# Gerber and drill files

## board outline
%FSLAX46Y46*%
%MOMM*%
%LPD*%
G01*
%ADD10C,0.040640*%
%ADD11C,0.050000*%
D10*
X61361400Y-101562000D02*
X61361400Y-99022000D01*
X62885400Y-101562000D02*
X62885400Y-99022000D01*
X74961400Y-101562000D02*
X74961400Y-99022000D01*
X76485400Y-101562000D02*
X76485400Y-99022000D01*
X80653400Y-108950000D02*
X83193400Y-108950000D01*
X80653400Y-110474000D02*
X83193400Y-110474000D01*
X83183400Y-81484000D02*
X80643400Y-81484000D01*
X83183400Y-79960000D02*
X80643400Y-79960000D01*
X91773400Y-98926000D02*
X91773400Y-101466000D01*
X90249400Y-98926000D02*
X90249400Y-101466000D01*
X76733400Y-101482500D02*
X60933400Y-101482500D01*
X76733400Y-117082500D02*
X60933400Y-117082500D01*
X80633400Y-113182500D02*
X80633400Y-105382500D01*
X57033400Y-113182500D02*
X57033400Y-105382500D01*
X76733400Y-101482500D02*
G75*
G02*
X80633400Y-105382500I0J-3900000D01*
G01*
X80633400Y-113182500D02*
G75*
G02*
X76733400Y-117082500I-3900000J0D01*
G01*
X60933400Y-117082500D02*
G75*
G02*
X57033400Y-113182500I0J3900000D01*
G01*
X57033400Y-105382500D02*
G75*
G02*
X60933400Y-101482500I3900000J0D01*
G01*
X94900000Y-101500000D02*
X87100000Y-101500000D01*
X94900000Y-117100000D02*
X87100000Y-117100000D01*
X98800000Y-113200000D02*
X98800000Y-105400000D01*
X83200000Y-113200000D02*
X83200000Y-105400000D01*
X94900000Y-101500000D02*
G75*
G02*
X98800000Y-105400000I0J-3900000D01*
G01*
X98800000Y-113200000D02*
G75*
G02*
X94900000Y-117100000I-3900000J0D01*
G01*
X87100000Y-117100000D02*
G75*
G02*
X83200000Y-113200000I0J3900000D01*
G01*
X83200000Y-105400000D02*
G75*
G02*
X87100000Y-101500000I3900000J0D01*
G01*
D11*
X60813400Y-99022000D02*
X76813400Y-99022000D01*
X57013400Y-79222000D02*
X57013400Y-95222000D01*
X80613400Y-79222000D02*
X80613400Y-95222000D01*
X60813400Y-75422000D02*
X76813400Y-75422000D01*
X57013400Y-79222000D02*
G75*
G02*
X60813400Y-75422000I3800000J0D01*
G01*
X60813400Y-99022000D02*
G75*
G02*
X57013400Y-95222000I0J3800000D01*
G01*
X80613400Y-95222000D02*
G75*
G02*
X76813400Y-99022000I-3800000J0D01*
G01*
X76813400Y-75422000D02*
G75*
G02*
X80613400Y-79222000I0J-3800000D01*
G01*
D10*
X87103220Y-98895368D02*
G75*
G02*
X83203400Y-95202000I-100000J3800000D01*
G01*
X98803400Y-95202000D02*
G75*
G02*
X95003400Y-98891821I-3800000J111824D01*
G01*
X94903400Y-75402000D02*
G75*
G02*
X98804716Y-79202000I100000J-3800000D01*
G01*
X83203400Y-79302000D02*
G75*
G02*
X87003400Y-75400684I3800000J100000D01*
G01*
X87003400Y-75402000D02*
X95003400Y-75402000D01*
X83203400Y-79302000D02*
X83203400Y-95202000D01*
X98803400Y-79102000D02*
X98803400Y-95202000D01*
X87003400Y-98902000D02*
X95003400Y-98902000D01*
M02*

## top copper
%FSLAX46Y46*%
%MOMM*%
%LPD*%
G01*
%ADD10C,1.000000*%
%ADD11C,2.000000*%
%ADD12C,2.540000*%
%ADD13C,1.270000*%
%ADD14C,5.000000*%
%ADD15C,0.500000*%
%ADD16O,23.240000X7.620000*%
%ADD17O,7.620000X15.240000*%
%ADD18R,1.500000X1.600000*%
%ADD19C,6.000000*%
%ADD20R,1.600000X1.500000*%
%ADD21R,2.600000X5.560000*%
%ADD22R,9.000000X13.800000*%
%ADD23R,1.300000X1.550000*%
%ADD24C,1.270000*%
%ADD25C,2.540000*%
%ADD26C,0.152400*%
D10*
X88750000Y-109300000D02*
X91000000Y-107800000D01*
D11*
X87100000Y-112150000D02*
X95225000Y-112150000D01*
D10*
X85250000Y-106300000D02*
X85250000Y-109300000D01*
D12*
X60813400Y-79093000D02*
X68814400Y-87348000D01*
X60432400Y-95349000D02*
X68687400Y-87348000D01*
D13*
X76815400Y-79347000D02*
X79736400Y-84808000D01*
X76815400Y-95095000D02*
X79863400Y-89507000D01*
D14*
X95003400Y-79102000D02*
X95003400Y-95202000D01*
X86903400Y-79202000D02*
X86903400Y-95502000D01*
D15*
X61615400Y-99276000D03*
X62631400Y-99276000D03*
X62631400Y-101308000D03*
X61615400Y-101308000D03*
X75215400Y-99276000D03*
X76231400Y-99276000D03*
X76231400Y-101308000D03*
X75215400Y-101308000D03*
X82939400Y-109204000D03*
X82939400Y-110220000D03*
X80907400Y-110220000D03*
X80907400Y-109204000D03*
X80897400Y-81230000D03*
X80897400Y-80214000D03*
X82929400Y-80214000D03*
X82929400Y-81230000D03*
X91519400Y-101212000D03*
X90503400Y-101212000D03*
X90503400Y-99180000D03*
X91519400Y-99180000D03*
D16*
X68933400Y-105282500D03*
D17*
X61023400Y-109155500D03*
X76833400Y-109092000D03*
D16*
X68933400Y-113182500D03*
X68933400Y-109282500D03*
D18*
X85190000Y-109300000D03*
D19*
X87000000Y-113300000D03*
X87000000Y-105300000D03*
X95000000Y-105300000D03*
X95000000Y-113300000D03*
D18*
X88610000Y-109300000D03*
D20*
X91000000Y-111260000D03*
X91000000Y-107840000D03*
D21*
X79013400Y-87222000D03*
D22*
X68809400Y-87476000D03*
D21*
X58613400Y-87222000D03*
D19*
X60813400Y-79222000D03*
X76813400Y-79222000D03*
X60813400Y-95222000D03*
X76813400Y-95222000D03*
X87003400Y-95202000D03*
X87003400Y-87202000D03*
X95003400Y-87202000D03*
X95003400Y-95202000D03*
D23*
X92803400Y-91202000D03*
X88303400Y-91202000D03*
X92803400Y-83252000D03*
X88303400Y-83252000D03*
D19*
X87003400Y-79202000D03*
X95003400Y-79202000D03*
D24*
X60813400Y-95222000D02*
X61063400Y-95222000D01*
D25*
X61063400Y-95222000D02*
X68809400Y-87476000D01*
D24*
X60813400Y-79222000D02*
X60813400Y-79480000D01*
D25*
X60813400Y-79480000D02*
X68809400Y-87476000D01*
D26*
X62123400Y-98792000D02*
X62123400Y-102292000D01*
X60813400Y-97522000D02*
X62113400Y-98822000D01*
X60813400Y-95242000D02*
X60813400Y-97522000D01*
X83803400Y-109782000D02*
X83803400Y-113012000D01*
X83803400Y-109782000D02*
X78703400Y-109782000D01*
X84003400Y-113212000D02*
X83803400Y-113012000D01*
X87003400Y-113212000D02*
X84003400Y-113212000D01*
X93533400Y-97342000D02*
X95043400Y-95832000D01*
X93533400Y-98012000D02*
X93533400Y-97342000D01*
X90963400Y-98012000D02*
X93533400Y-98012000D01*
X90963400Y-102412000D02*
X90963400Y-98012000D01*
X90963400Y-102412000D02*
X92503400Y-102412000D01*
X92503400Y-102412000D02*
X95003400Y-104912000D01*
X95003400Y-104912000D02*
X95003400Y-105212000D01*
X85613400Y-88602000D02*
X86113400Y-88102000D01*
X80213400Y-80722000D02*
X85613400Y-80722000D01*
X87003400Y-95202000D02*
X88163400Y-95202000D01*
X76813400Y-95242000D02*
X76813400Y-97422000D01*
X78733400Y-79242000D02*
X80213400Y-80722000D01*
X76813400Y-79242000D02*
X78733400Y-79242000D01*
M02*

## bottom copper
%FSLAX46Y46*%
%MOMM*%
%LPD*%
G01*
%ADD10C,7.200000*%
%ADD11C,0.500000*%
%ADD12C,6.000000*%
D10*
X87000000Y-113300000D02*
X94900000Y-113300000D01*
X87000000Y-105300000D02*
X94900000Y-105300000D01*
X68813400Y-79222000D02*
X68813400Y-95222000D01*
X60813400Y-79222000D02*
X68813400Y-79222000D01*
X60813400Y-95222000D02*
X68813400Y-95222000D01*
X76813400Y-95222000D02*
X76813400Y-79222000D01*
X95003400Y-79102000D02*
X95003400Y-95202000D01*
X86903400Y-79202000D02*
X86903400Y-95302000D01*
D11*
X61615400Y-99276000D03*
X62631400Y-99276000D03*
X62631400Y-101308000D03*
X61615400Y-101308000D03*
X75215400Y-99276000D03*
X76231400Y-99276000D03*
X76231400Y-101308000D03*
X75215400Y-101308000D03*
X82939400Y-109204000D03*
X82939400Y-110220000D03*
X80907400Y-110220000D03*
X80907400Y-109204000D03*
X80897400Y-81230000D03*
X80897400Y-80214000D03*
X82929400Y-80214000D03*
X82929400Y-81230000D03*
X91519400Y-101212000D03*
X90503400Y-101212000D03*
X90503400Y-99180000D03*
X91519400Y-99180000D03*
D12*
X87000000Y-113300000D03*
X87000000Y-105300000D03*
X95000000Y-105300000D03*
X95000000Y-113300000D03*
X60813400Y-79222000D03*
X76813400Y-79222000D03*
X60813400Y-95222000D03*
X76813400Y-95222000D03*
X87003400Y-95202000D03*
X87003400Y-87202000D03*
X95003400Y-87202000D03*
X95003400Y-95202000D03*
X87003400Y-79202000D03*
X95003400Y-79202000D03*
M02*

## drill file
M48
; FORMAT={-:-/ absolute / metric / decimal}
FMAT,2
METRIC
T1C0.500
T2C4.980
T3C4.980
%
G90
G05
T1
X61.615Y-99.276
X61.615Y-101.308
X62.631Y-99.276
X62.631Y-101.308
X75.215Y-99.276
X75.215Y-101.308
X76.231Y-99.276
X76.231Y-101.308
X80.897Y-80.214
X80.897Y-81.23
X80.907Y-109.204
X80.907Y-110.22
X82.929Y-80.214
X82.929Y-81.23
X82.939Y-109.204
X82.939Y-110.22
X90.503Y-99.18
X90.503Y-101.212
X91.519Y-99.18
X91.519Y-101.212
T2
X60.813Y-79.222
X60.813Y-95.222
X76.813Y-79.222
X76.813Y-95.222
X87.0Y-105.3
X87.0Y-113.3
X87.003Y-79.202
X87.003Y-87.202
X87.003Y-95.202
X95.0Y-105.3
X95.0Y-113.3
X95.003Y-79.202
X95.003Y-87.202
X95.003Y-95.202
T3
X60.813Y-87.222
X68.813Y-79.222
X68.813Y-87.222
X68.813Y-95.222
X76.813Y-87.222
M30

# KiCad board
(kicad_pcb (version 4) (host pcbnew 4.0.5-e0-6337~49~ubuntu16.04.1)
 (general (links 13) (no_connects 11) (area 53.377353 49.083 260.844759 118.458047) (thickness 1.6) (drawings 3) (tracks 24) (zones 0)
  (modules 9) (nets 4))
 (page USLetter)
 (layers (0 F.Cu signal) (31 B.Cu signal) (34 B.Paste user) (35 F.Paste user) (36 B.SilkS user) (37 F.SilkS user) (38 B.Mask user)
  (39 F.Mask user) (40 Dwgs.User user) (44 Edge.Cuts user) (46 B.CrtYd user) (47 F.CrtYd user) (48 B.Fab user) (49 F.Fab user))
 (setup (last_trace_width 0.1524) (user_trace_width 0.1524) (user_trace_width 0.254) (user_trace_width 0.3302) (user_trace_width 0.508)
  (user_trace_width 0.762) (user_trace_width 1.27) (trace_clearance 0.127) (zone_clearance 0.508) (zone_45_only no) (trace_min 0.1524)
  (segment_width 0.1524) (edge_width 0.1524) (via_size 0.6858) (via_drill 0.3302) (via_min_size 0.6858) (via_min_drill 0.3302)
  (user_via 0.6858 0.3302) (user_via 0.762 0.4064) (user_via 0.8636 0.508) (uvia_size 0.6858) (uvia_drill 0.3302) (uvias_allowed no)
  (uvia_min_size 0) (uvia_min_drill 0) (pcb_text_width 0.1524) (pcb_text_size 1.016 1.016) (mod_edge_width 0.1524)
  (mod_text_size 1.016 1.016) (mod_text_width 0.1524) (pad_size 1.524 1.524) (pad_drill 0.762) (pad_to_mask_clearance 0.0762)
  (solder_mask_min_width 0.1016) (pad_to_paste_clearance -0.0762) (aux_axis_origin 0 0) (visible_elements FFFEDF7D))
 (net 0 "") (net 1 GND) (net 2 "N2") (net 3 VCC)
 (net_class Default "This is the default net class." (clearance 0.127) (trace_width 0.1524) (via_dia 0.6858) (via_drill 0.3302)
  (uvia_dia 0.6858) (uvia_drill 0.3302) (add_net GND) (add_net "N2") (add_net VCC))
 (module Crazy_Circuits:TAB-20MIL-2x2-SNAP (layer F.Cu) (at 62.1234 100.292)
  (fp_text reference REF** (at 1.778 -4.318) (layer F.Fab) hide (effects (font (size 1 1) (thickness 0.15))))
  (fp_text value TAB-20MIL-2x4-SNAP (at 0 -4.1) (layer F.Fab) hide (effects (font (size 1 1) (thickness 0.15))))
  (fp_line (start -0.762 1.27) (end -0.762 -1.27) (layer Edge.Cuts) (width 0.04064))
  (fp_line (start 0.762 1.27) (end 0.762 -1.27) (layer Edge.Cuts) (width 0.04064))
  (pad 1 thru_hole circle (at -0.508 -1.016) (size 0.5 0.5) (drill 0.5) (layers *.Cu))
  (pad 1 thru_hole circle (at 0.508 -1.016) (size 0.5 0.5) (drill 0.5) (layers *.Cu))
  (pad 1 thru_hole circle (at 0.508 1.016) (size 0.5 0.5) (drill 0.5) (layers *.Cu))
  (pad 1 thru_hole circle (at -0.508 1.016) (size 0.5 0.5) (drill 0.5) (layers *.Cu)))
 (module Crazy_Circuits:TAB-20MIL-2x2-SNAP (layer F.Cu) (at 75.7234 100.292)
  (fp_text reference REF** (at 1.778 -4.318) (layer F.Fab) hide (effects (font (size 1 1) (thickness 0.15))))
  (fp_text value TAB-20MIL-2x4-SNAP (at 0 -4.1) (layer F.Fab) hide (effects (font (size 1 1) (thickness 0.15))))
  (fp_line (start -0.762 1.27) (end -0.762 -1.27) (layer Edge.Cuts) (width 0.04064))
  (fp_line (start 0.762 1.27) (end 0.762 -1.27) (layer Edge.Cuts) (width 0.04064))
  (pad 1 thru_hole circle (at -0.508 -1.016) (size 0.5 0.5) (drill 0.5) (layers *.Cu))
  (pad 1 thru_hole circle (at 0.508 -1.016) (size 0.5 0.5) (drill 0.5) (layers *.Cu))
  (pad 1 thru_hole circle (at 0.508 1.016) (size 0.5 0.5) (drill 0.5) (layers *.Cu))
  (pad 1 thru_hole circle (at -0.508 1.016) (size 0.5 0.5) (drill 0.5) (layers *.Cu)))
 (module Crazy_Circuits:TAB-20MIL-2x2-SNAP (layer F.Cu) (at 81.9234 109.712 270)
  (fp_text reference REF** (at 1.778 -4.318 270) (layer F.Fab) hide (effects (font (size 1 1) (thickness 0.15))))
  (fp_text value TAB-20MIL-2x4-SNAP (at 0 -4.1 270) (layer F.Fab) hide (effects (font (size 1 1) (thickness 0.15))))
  (fp_line (start -0.762 1.27) (end -0.762 -1.27) (layer Edge.Cuts) (width 0.04064))
  (fp_line (start 0.762 1.27) (end 0.762 -1.27) (layer Edge.Cuts) (width 0.04064))
  (pad 1 thru_hole circle (at -0.508 -1.016 270) (size 0.5 0.5) (drill 0.5) (layers *.Cu))
  (pad 1 thru_hole circle (at 0.508 -1.016 270) (size 0.5 0.5) (drill 0.5) (layers *.Cu))
  (pad 1 thru_hole circle (at 0.508 1.016 270) (size 0.5 0.5) (drill 0.5) (layers *.Cu))
  (pad 1 thru_hole circle (at -0.508 1.016 270) (size 0.5 0.5) (drill 0.5) (layers *.Cu)))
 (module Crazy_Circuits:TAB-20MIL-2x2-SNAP (layer F.Cu) (at 81.9134 80.722 90)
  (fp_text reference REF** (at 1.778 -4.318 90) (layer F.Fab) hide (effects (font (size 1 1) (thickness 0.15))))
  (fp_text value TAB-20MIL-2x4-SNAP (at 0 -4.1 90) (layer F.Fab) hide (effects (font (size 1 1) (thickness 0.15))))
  (fp_line (start -0.762 1.27) (end -0.762 -1.27) (layer Edge.Cuts) (width 0.04064))
  (fp_line (start 0.762 1.27) (end 0.762 -1.27) (layer Edge.Cuts) (width 0.04064))
  (pad 1 thru_hole circle (at -0.508 -1.016 90) (size 0.5 0.5) (drill 0.5) (layers *.Cu))
  (pad 1 thru_hole circle (at 0.508 -1.016 90) (size 0.5 0.5) (drill 0.5) (layers *.Cu))
  (pad 1 thru_hole circle (at 0.508 1.016 90) (size 0.5 0.5) (drill 0.5) (layers *.Cu))
  (pad 1 thru_hole circle (at -0.508 1.016 90) (size 0.5 0.5) (drill 0.5) (layers *.Cu)))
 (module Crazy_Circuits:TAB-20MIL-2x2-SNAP (layer F.Cu) (at 91.0114 100.196 180)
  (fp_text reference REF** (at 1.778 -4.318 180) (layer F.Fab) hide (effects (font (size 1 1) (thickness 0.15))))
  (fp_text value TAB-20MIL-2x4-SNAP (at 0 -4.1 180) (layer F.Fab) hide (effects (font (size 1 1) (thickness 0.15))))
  (fp_line (start -0.762 1.27) (end -0.762 -1.27) (layer Edge.Cuts) (width 0.04064))
  (fp_line (start 0.762 1.27) (end 0.762 -1.27) (layer Edge.Cuts) (width 0.04064))
  (pad 1 thru_hole circle (at -0.508 -1.016 180) (size 0.5 0.5) (drill 0.5) (layers *.Cu))
  (pad 1 thru_hole circle (at 0.508 -1.016 180) (size 0.5 0.5) (drill 0.5) (layers *.Cu))
  (pad 1 thru_hole circle (at 0.508 1.016 180) (size 0.5 0.5) (drill 0.5) (layers *.Cu))
  (pad 1 thru_hole circle (at -0.508 1.016 180) (size 0.5 0.5) (drill 0.5) (layers *.Cu)))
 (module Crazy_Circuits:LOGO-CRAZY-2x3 (layer F.Cu) (at 64.8334 109.2825)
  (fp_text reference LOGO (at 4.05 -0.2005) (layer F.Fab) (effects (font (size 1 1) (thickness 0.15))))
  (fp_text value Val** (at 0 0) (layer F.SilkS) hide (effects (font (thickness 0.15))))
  (fp_line (start 11.9 -7.8) (end -3.9 -7.8) (layer Edge.Cuts) (width 0.04064))
  (fp_line (start 11.9 7.8) (end -3.9 7.8) (layer Edge.Cuts) (width 0.04064))
  (fp_line (start 15.8 3.9) (end 15.8 -3.9) (layer Edge.Cuts) (width 0.04064))
  (fp_line (start -7.8 3.9) (end -7.8 -3.9) (layer Edge.Cuts) (width 0.04064))
  (fp_arc (start 11.9 -3.9) (end 11.9 -7.8) (angle 90) (layer Edge.Cuts) (width 0.04064))
  (fp_arc (start 11.9 3.9) (end 15.8 3.9) (angle 90) (layer Edge.Cuts) (width 0.04064))
  (fp_arc (start -3.9 3.9) (end -3.9 7.8) (angle 90) (layer Edge.Cuts) (width 0.04064))
  (fp_arc (start -3.9 -3.9) (end -7.8 -3.9) (angle 90) (layer Edge.Cuts) (width 0.04064))
  (pad BG smd oval (at 4.1 -4) (size 23.24 7.62) (layers F.Cu))
  (pad BG smd oval (at -3.81 -0.127 90) (size 15.24 7.62) (layers F.Cu))
  (pad BG smd oval (at 12 -0.1905 270) (size 15.24 7.62) (layers F.Cu))
  (pad BG smd oval (at 4.1 3.9) (size 23.24 7.62) (layers F.Cu)) (pad BG smd oval (at 4.1 0) (size 23.24 7.62) (layers F.Cu)))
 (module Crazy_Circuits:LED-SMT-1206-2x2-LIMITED (layer F.Cu) (at 87 113.3)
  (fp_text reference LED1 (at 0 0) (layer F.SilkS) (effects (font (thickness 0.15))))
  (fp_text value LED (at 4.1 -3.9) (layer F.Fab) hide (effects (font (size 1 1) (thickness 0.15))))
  (fp_line (start 1.75 -4) (end 4 -5.5) (layer F.Cu) (width 1)) (fp_line (start 0 0) (end 7.9 0) (layer B.Cu) (width 7.2))
  (fp_line (start 0 -8) (end 7.9 -8) (layer B.Cu) (width 7.2))
  (fp_line (start 0.1 -1.15) (end 8.225 -1.15) (layer F.Cu) (width 2))
  (fp_line (start 7.9 -11.8) (end 0.1 -11.8) (layer Edge.Cuts) (width 0.04064))
  (fp_line (start 7.9 3.8) (end 0.1 3.8) (layer Edge.Cuts) (width 0.04064))
  (fp_line (start 11.8 -0.1) (end 11.8 -7.9) (layer Edge.Cuts) (width 0.04064))
  (fp_line (start -3.8 -0.1) (end -3.8 -7.9) (layer Edge.Cuts) (width 0.04064))
  (fp_arc (start 7.9 -7.9) (end 7.9 -11.8) (angle 90) (layer Edge.Cuts) (width 0.04064))
  (fp_arc (start 7.9 -0.1) (end 11.8 -0.1) (angle 90) (layer Edge.Cuts) (width 0.04064))
  (fp_arc (start 0.1 -0.1) (end 0.1 3.8) (angle 90) (layer Edge.Cuts) (width 0.04064))
  (fp_arc (start 0.1 -7.9) (end -3.8 -7.9) (angle 90) (layer Edge.Cuts) (width 0.04064))
  (fp_line (start -1.75 -7) (end -1.75 -4) (layer F.Cu) (width 1))
  (pad 1 smd rect (at -1.81 -4 90) (size 1.6 1.5) (layers F.Cu F.Paste F.Mask))
  (pad - thru_hole circle (at 0 0) (size 6 6) (drill 4.98) (layers *.Cu B.Mask) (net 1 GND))
  (pad + thru_hole circle (at 0 -8) (size 6 6) (drill 4.98) (layers *.Cu B.Mask) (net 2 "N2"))
  (pad + thru_hole circle (at 8 -8) (size 6 6) (drill 4.98) (layers *.Cu B.Mask) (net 2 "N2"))
  (pad - thru_hole circle (at 8 0) (size 6 6) (drill 4.98) (layers *.Cu B.Mask) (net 1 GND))
  (pad 3 smd rect (at 1.61 -4 90) (size 1.6 1.5) (layers F.Cu F.Paste F.Mask))
  (pad 2 smd rect (at 4 -2.04) (size 1.6 1.5) (layers F.Cu F.Paste F.Mask))
  (pad 3 smd rect (at 4 -5.46) (size 1.6 1.5) (layers F.Cu F.Paste F.Mask)))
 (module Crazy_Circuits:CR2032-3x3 (layer F.Cu) (at 60.8134 95.222)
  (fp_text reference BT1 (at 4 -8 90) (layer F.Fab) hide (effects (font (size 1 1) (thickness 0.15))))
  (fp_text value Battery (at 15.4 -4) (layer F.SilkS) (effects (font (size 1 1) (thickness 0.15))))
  (fp_line (start 0 -16.129) (end 8.001 -7.874) (layer F.Cu) (width 2.54))
  (fp_line (start 0 3.8) (end 16 3.8) (layer Edge.Cuts) (width 0.05))
  (fp_line (start -3.8 -16) (end -3.8 0) (layer Edge.Cuts) (width 0.05))
  (fp_line (start 19.8 -16) (end 19.8 0) (layer Edge.Cuts) (width 0.05))
  (fp_line (start 0 -19.8) (end 16 -19.8) (layer Edge.Cuts) (width 0.05))
  (fp_arc (start 0 -16) (end -3.8 -16) (angle 90) (layer Edge.Cuts) (width 0.05))
  (fp_arc (start 0 0) (end 0 3.8) (angle 90) (layer Edge.Cuts) (width 0.05))
  (fp_arc (start 16 0) (end 19.8 0) (angle 90) (layer Edge.Cuts) (width 0.05))
  (fp_arc (start 16 -16) (end 16 -19.8) (angle 90) (layer Edge.Cuts) (width 0.05))
  (fp_line (start 8 -16) (end 8 0) (layer B.Cu) (width 7.2)) (fp_line (start 0 -16) (end 8 -16) (layer B.Cu) (width 7.2))
  (fp_line (start 0 0) (end 8 0) (layer B.Cu) (width 7.2)) (fp_line (start 16 0) (end 16 -16) (layer B.Cu) (width 7.2))
  (fp_line (start -0.381 0.127) (end 7.874 -7.874) (layer F.Cu) (width 2.54))
  (fp_line (start 16.002 -15.875) (end 18.923 -10.414) (layer F.Cu) (width 1.27))
  (fp_line (start 16.002 -0.127) (end 19.05 -5.715) (layer F.Cu) (width 1.27))
  (pad "" np_thru_hole circle (at 8 -8) (size 4.98 4.98) (drill 4.98) (layers *.Cu B.Mask))
  (pad "" np_thru_hole circle (at 0 -8) (size 4.98 4.98) (drill 4.98) (layers *.Cu B.Mask))
  (pad "" np_thru_hole circle (at 16 -8) (size 4.98 4.98) (drill 4.98) (layers *.Cu B.Mask))
  (pad + smd rect (at 18.2 -8) (size 2.6 5.56) (layers F.Cu F.Paste F.Mask) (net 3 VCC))
  (pad GND smd rect (at 7.996 -7.746) (size 9 13.8) (layers F.Cu F.Paste F.Mask) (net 1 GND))
  (pad + smd rect (at -2.2 -8) (size 2.6 5.56) (layers F.Cu F.Paste F.Mask) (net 3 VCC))
  (pad GND thru_hole circle (at 0 -16) (size 6 6) (drill 4.98) (layers *.Cu B.Mask) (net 1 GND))
  (pad "" np_thru_hole circle (at 8 -16) (size 4.98 4.98) (drill 4.98) (layers *.Cu B.Mask))
  (pad + thru_hole circle (at 16 -16) (size 6 6) (drill 4.98) (layers *.Cu B.Mask) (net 3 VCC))
  (pad GND thru_hole circle (at 0 0) (size 6 6) (drill 4.98) (layers *.Cu B.Mask) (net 1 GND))
  (pad "" np_thru_hole circle (at 8 0) (size 4.98 4.98) (drill 4.98) (layers *.Cu B.Mask))
  (pad + thru_hole circle (at 16 0) (size 6 6) (drill 4.98) (layers *.Cu B.Mask) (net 3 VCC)))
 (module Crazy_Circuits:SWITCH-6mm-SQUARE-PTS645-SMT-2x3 (layer F.Cu) (at 95.0034 95.202 90)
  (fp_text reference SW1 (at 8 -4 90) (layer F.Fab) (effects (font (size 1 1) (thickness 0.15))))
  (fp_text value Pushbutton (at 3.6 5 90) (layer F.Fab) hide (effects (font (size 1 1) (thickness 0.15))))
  (fp_arc (start 0.106632 -8.00018) (end -3.693368 -7.90018) (angle 89.9) (layer Edge.Cuts) (width 0.04064))
  (fp_arc (start 0.111824 0) (end 0 3.8) (angle 88.31442243) (layer Edge.Cuts) (width 0.04064))
  (fp_arc (start 16 0) (end 19.8 -0.1) (angle 91.50743576) (layer Edge.Cuts) (width 0.04064))
  (fp_arc (start 16 -8) (end 15.9 -11.8) (angle 91.50743576) (layer Edge.Cuts) (width 0.04064))
  (fp_line (start 19.8 -8) (end 19.8 0) (layer Edge.Cuts) (width 0.04064))
  (fp_line (start 15.9 -11.8) (end 0 -11.8) (layer Edge.Cuts) (width 0.04064))
  (fp_line (start 16.1 3.8) (end 0 3.8) (layer Edge.Cuts) (width 0.04064))
  (fp_line (start -3.7 -8) (end -3.7 0) (layer Edge.Cuts) (width 0.04064)) (fp_line (start 16.1 0) (end 0 0) (layer B.Cu) (width 7.2))
  (fp_line (start 16.1 0) (end 0 0) (layer F.Cu) (width 5))
  (fp_line (start 16 -8.1) (end -0.3 -8.1) (layer F.Cu) (width 5))
  (fp_line (start 16 -8.1) (end -0.1 -8.1) (layer B.Cu) (width 7.2))
  (pad 1 thru_hole circle (at 0 -8) (size 6 6) (drill 4.98) (layers *.Cu B.Mask) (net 3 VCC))
  (pad 2 thru_hole circle (at 8 -8) (size 6 6) (drill 4.98) (layers *.Cu B.Mask) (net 2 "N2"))
  (pad 4 thru_hole circle (at 8 0) (size 6 6) (drill 4.98) (layers *.Cu B.Mask))
  (pad 3 thru_hole circle (at 0 0) (size 6 6) (drill 4.98) (layers *.Cu B.Mask))
  (pad 3 smd rect (at 4 -2.2 90) (size 1.55 1.3) (layers F.Cu F.Paste F.Mask) (solder_mask_margin 0.0762))
  (pad 1 smd rect (at 4 -6.7 90) (size 1.55 1.3) (layers F.Cu F.Paste F.Mask) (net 3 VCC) (solder_mask_margin 0.0762))
  (pad 4 smd rect (at 11.95 -2.2 90) (size 1.55 1.3) (layers F.Cu F.Paste F.Mask) (solder_mask_margin 0.0762))
  (pad 2 smd rect (at 11.95 -6.7 90) (size 1.55 1.3) (layers F.Cu F.Paste F.Mask) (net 2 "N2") (solder_mask_margin 0.0762))
  (pad 2 thru_hole circle (at 16 -8) (size 6 6) (drill 4.98) (layers *.Cu B.Mask) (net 2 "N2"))
  (pad 4 thru_hole circle (at 16 0) (size 6 6) (drill 4.98) (layers *.Cu B.Mask)))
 (segment (start 60.8134 95.222) (end 61.0634 95.222) (width 1.27) (layer F.Cu) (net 1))
 (segment (start 61.0634 95.222) (end 68.8094 87.476) (width 2.54) (layer F.Cu) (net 1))
 (segment (start 60.8134 79.222) (end 60.8134 79.48) (width 1.27) (layer F.Cu) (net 1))
 (segment (start 60.8134 79.48) (end 68.8094 87.476) (width 2.54) (layer F.Cu) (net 1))
 (segment (start 62.1234 98.792) (end 62.1234 102.292) (width 0.1524) (layer F.Cu) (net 1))
 (segment (start 60.8134 97.522) (end 62.1134 98.822) (width 0.1524) (layer F.Cu) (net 1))
 (segment (start 60.8134 95.242) (end 60.8134 97.522) (width 0.1524) (layer F.Cu) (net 1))
 (segment (start 83.8034 109.782) (end 83.8034 113.012) (width 0.1524) (layer F.Cu) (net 1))
 (segment (start 83.8034 109.782) (end 78.7034 109.782) (width 0.1524) (layer F.Cu) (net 1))
 (segment (start 84.0034 113.212) (end 83.8034 113.012) (width 0.1524) (layer F.Cu) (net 1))
 (segment (start 87.0034 113.212) (end 84.0034 113.212) (width 0.1524) (layer F.Cu) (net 1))
 (segment (start 93.5334 97.342) (end 95.0434 95.832) (width 0.1524) (layer F.Cu) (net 2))
 (segment (start 93.5334 98.012) (end 93.5334 97.342) (width 0.1524) (layer F.Cu) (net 2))
 (segment (start 90.9634 98.012) (end 93.5334 98.012) (width 0.1524) (layer F.Cu) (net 2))
 (segment (start 90.9634 102.412) (end 90.9634 98.012) (width 0.1524) (layer F.Cu) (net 2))
 (segment (start 90.9634 102.412) (end 92.5034 102.412) (width 0.1524) (layer F.Cu) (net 2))
 (segment (start 92.5034 102.412) (end 95.0034 104.912) (width 0.1524) (layer F.Cu) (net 2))
 (segment (start 95.0034 104.912) (end 95.0034 105.212) (width 0.1524) (layer F.Cu) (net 2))
 (segment (start 85.6134 88.602) (end 86.1134 88.102) (width 0.1524) (layer F.Cu) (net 2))
 (segment (start 80.2134 80.722) (end 85.6134 80.722) (width 0.1524) (layer F.Cu) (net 2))
 (segment (start 87.0034 95.202) (end 88.1634 95.202) (width 0.1524) (layer F.Cu) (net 3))
 (segment (start 76.8134 95.242) (end 76.8134 97.422) (width 0.1524) (layer F.Cu) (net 3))
 (segment (start 78.7334 79.242) (end 80.2134 80.722) (width 0.1524) (layer F.Cu) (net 3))
 (segment (start 76.8134 79.242) (end 78.7334 79.242) (width 0.1524) (layer F.Cu) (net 3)))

